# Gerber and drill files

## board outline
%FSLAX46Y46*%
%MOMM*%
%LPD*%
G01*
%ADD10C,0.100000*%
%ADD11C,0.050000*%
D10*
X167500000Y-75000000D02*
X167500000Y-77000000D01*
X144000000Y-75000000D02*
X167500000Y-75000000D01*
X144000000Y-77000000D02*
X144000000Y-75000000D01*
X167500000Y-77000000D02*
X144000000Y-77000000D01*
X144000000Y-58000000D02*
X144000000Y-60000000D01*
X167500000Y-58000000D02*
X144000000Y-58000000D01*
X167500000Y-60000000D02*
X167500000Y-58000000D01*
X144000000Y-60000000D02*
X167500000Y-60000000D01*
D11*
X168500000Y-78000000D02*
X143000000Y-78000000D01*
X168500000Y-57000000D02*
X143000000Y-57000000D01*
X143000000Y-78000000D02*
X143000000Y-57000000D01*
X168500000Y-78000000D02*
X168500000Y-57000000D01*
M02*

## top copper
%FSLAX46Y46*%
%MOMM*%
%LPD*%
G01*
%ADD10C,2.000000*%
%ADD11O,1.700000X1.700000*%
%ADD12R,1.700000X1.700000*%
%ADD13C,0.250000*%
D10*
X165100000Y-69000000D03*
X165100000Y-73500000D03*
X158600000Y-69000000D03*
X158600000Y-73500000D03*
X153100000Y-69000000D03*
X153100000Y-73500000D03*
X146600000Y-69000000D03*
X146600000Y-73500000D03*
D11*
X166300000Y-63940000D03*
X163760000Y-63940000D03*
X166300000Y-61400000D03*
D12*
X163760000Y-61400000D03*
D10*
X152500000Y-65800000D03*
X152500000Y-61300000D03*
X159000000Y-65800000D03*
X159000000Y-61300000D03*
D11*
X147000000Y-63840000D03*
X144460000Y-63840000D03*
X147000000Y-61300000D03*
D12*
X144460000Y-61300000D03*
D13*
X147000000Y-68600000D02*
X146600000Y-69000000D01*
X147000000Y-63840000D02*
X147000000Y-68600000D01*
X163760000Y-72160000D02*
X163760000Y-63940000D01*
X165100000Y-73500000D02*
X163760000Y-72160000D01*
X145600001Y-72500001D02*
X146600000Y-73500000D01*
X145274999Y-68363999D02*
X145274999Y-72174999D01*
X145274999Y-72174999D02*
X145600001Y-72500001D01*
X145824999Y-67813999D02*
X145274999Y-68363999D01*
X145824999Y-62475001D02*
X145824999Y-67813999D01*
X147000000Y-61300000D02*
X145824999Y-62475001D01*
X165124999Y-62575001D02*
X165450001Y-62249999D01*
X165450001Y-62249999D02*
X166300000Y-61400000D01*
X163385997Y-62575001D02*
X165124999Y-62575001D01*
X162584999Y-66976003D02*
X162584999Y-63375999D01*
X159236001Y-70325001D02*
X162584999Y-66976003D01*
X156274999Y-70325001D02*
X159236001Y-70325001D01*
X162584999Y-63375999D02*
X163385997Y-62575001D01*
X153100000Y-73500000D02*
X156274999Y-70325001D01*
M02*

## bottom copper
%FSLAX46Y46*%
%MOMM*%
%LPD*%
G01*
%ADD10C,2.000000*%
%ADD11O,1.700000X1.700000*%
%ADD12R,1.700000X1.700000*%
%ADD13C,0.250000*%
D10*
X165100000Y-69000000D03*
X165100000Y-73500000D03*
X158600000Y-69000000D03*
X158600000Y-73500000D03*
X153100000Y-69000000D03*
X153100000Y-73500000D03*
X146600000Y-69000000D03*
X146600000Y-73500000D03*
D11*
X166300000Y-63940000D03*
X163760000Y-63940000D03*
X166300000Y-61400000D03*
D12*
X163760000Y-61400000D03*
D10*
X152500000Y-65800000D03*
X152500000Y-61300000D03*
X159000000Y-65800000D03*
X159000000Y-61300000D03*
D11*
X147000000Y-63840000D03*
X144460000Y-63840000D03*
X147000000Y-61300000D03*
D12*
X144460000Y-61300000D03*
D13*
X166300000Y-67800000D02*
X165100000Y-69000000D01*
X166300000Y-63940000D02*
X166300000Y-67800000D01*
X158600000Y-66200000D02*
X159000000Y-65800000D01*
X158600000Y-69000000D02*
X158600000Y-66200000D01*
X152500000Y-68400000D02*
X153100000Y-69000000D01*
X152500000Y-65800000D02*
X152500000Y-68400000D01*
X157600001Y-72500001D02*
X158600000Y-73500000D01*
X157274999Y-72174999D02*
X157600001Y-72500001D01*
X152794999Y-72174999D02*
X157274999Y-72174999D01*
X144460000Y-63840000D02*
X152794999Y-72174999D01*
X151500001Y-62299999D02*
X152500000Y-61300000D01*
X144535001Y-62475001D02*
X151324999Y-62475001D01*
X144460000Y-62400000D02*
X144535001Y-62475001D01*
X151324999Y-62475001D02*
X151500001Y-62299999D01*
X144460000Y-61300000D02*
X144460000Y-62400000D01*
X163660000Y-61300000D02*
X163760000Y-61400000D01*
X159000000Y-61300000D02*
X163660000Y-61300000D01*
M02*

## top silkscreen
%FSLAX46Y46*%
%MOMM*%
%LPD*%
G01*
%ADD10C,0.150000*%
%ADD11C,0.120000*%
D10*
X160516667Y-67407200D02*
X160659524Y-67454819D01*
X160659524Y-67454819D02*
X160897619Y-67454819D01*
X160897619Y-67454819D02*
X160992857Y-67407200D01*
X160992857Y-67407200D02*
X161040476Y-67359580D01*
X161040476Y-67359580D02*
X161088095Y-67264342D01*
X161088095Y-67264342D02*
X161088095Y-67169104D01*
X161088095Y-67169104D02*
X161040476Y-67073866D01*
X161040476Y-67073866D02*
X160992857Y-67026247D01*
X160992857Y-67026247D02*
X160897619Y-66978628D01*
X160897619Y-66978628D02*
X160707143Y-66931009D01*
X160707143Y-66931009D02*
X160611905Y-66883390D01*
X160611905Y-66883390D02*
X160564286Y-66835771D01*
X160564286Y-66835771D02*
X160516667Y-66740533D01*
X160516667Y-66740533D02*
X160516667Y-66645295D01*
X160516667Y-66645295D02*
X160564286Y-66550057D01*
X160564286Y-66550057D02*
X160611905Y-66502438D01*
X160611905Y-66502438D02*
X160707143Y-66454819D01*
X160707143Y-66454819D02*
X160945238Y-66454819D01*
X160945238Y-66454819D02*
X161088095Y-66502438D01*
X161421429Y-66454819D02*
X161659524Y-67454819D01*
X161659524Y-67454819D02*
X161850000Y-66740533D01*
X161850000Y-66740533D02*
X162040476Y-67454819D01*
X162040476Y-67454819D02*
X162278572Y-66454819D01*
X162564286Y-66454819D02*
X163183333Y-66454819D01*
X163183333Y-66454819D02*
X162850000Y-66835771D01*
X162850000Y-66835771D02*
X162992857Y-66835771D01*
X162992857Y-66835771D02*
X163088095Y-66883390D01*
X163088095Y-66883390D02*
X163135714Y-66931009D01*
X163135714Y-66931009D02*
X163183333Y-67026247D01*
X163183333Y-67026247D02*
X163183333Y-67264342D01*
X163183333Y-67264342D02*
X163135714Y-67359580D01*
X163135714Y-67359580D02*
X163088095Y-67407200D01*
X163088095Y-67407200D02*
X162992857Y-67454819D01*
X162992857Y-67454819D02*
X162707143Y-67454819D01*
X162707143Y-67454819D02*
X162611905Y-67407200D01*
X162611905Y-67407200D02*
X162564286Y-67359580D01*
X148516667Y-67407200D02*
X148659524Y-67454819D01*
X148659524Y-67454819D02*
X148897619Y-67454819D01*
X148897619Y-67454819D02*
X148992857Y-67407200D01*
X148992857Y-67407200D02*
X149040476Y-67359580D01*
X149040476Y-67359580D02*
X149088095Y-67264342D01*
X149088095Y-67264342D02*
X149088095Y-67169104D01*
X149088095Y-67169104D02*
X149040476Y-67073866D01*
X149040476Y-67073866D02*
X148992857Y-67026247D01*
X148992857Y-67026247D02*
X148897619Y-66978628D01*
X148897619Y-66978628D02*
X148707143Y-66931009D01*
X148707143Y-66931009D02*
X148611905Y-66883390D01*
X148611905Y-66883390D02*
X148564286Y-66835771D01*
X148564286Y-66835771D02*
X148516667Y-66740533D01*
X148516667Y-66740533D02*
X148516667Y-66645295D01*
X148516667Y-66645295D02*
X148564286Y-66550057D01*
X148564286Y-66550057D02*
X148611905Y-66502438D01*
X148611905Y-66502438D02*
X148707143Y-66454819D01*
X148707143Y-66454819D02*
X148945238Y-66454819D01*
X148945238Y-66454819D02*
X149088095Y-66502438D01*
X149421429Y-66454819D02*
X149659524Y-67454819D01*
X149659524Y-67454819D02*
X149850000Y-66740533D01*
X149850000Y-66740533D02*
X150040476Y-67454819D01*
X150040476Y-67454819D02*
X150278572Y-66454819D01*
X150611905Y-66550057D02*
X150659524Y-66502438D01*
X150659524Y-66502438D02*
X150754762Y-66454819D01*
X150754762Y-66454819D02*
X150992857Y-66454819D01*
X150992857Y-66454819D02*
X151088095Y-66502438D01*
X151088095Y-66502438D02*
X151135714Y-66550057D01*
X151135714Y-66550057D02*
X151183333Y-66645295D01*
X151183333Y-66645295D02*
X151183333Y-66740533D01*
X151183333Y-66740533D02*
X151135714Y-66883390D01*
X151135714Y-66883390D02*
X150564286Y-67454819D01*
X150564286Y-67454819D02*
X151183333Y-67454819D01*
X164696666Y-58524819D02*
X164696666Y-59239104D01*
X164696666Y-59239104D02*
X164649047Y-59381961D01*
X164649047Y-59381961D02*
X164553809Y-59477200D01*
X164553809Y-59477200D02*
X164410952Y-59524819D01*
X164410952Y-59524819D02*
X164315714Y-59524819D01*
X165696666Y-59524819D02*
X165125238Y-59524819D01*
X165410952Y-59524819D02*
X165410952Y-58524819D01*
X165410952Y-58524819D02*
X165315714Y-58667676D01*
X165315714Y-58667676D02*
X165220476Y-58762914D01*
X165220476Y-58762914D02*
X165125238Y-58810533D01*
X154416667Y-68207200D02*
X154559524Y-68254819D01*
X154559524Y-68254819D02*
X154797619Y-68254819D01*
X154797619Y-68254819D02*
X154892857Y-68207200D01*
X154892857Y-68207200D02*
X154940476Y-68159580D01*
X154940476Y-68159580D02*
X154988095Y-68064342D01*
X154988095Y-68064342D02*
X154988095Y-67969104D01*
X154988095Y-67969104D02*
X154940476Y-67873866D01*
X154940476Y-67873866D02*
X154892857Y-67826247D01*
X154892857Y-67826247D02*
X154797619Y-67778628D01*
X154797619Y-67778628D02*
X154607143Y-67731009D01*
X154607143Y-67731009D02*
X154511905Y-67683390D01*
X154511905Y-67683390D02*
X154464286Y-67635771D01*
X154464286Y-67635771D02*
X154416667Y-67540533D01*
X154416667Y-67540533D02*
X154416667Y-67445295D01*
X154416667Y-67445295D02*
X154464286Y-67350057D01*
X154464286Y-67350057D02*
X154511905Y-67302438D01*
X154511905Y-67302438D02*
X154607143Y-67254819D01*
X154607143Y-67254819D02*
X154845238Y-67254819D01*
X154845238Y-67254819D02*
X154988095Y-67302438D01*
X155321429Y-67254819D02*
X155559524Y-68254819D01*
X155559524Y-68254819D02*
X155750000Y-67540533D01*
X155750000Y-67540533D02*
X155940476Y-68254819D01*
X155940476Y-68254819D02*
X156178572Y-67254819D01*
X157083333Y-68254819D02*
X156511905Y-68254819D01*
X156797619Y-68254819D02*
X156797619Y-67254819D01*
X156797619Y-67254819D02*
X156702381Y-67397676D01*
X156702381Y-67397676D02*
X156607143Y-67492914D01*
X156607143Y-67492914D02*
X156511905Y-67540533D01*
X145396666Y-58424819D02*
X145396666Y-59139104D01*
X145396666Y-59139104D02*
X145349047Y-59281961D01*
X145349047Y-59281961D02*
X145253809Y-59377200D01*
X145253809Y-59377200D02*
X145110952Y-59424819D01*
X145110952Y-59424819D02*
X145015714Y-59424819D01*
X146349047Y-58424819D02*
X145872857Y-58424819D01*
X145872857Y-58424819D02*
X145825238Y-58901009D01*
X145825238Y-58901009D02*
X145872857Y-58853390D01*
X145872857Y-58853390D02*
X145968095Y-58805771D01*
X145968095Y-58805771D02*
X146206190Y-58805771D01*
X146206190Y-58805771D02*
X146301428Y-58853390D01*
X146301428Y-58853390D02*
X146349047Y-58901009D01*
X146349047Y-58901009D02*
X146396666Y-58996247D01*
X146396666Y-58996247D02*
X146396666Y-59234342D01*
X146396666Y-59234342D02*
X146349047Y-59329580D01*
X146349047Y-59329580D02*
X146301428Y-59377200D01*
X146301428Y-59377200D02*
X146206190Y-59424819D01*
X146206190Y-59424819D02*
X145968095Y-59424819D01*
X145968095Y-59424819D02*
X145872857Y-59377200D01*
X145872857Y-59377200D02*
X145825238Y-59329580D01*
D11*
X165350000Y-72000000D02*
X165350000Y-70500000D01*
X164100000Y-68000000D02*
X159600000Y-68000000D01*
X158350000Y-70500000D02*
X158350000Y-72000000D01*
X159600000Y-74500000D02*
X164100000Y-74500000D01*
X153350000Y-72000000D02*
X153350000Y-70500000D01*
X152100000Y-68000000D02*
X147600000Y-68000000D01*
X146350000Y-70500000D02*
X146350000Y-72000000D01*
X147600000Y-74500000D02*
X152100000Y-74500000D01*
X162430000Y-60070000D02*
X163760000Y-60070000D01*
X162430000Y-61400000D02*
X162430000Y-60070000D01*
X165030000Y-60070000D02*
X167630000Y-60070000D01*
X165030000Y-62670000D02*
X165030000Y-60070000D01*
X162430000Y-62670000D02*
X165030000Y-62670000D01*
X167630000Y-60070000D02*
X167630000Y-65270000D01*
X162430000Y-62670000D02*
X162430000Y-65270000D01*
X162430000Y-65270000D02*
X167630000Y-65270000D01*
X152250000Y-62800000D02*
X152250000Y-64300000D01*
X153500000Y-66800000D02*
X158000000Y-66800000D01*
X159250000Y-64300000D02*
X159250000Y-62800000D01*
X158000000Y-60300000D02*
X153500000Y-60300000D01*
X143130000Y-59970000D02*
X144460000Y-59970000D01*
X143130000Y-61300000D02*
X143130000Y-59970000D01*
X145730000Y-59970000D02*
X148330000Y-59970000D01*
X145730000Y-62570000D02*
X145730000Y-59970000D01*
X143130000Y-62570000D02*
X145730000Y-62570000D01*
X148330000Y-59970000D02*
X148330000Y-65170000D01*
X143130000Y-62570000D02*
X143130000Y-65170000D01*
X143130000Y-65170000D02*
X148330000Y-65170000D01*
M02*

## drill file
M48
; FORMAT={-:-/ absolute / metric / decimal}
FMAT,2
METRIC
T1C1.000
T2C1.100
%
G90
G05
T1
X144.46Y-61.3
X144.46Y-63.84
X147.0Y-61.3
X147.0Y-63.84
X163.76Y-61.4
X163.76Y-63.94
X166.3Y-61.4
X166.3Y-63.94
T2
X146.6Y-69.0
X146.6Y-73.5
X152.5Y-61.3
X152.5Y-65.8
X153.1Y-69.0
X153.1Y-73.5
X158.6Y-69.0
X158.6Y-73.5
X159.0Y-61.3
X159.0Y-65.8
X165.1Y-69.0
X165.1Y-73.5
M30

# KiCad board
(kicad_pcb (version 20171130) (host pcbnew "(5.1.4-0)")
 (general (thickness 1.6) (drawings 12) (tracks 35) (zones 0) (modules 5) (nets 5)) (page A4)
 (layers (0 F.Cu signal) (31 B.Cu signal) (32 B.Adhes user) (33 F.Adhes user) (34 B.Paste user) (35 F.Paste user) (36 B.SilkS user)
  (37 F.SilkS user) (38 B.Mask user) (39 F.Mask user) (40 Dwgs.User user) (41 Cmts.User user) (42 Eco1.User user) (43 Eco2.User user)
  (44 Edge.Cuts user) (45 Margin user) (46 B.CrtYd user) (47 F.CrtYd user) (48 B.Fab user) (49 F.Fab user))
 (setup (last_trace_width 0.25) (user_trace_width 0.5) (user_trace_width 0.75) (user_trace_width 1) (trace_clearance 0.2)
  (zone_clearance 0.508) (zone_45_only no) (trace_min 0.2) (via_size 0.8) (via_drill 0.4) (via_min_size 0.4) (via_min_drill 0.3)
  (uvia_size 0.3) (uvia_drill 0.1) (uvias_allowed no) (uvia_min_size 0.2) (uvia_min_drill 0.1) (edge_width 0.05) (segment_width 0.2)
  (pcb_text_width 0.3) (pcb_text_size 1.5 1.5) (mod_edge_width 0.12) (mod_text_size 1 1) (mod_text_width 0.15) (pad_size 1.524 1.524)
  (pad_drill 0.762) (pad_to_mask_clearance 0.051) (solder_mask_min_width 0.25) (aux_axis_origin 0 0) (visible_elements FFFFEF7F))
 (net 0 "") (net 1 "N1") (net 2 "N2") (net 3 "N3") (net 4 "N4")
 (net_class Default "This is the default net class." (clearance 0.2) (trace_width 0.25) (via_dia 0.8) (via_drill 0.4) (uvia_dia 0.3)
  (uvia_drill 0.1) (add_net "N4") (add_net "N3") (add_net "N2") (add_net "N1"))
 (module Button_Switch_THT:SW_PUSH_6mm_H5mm (layer F.Cu) (at 158.6 69)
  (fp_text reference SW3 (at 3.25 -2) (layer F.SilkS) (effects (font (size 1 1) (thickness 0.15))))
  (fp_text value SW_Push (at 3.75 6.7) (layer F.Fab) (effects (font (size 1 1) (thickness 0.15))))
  (fp_line (start 6.75 3) (end 6.75 1.5) (layer F.SilkS) (width 0.12))
  (fp_line (start 5.5 -1) (end 1 -1) (layer F.SilkS) (width 0.12))
  (fp_line (start -0.25 1.5) (end -0.25 3) (layer F.SilkS) (width 0.12))
  (fp_line (start 1 5.5) (end 5.5 5.5) (layer F.SilkS) (width 0.12))
  (pad 1 thru_hole circle (at 6.5 0 90) (size 2 2) (drill 1.1) (layers *.Cu *.Mask) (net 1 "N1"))
  (pad 2 thru_hole circle (at 6.5 4.5 90) (size 2 2) (drill 1.1) (layers *.Cu *.Mask) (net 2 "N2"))
  (pad 1 thru_hole circle (at 0 0 90) (size 2 2) (drill 1.1) (layers *.Cu *.Mask) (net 1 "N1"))
  (pad 2 thru_hole circle (at 0 4.5 90) (size 2 2) (drill 1.1) (layers *.Cu *.Mask) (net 2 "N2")))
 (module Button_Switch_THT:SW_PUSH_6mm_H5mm (layer F.Cu) (at 146.6 69)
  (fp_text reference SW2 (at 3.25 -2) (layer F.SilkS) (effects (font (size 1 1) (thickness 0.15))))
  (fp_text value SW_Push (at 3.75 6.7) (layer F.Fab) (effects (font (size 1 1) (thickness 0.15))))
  (fp_line (start 6.75 3) (end 6.75 1.5) (layer F.SilkS) (width 0.12))
  (fp_line (start 5.5 -1) (end 1 -1) (layer F.SilkS) (width 0.12))
  (fp_line (start -0.25 1.5) (end -0.25 3) (layer F.SilkS) (width 0.12))
  (fp_line (start 1 5.5) (end 5.5 5.5) (layer F.SilkS) (width 0.12))
  (pad 1 thru_hole circle (at 6.5 0 90) (size 2 2) (drill 1.1) (layers *.Cu *.Mask) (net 1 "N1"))
  (pad 2 thru_hole circle (at 6.5 4.5 90) (size 2 2) (drill 1.1) (layers *.Cu *.Mask) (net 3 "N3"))
  (pad 1 thru_hole circle (at 0 0 90) (size 2 2) (drill 1.1) (layers *.Cu *.Mask) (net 1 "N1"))
  (pad 2 thru_hole circle (at 0 4.5 90) (size 2 2) (drill 1.1) (layers *.Cu *.Mask) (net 3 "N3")))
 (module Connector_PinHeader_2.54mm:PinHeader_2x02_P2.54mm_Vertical (layer F.Cu) (at 163.76 61.4)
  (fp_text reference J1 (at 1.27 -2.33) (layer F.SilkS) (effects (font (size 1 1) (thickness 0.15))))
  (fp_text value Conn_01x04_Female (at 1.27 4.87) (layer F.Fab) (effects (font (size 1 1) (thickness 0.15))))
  (fp_line (start -1.33 -1.33) (end 0 -1.33) (layer F.SilkS) (width 0.12))
  (fp_line (start -1.33 0) (end -1.33 -1.33) (layer F.SilkS) (width 0.12))
  (fp_line (start 1.27 -1.33) (end 3.87 -1.33) (layer F.SilkS) (width 0.12))
  (fp_line (start 1.27 1.27) (end 1.27 -1.33) (layer F.SilkS) (width 0.12))
  (fp_line (start -1.33 1.27) (end 1.27 1.27) (layer F.SilkS) (width 0.12))
  (fp_line (start 3.87 -1.33) (end 3.87 3.87) (layer F.SilkS) (width 0.12))
  (fp_line (start -1.33 1.27) (end -1.33 3.87) (layer F.SilkS) (width 0.12))
  (fp_line (start -1.33 3.87) (end 3.87 3.87) (layer F.SilkS) (width 0.12))
  (pad 4 thru_hole oval (at 2.54 2.54) (size 1.7 1.7) (drill 1) (layers *.Cu *.Mask) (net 1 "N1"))
  (pad 3 thru_hole oval (at 0 2.54) (size 1.7 1.7) (drill 1) (layers *.Cu *.Mask) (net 2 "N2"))
  (pad 2 thru_hole oval (at 2.54 0) (size 1.7 1.7) (drill 1) (layers *.Cu *.Mask) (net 3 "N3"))
  (pad 1 thru_hole rect (at 0 0) (size 1.7 1.7) (drill 1) (layers *.Cu *.Mask) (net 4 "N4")))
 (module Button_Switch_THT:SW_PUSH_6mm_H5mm (layer F.Cu) (at 159 65.8 180)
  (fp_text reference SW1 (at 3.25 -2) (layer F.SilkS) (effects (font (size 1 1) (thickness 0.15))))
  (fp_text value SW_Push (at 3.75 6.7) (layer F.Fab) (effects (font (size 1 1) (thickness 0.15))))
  (fp_line (start 6.75 3) (end 6.75 1.5) (layer F.SilkS) (width 0.12))
  (fp_line (start 5.5 -1) (end 1 -1) (layer F.SilkS) (width 0.12))
  (fp_line (start -0.25 1.5) (end -0.25 3) (layer F.SilkS) (width 0.12))
  (fp_line (start 1 5.5) (end 5.5 5.5) (layer F.SilkS) (width 0.12))
  (pad 1 thru_hole circle (at 6.5 0 270) (size 2 2) (drill 1.1) (layers *.Cu *.Mask) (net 1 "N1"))
  (pad 2 thru_hole circle (at 6.5 4.5 270) (size 2 2) (drill 1.1) (layers *.Cu *.Mask) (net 4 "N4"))
  (pad 1 thru_hole circle (at 0 0 270) (size 2 2) (drill 1.1) (layers *.Cu *.Mask) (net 1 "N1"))
  (pad 2 thru_hole circle (at 0 4.5 270) (size 2 2) (drill 1.1) (layers *.Cu *.Mask) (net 4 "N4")))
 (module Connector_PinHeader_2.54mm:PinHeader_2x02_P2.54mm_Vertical (layer F.Cu) (at 144.46 61.3)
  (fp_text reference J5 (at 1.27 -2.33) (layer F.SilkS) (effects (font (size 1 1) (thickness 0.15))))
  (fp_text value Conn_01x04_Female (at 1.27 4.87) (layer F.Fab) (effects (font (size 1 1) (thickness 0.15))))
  (fp_line (start -1.33 -1.33) (end 0 -1.33) (layer F.SilkS) (width 0.12))
  (fp_line (start -1.33 0) (end -1.33 -1.33) (layer F.SilkS) (width 0.12))
  (fp_line (start 1.27 -1.33) (end 3.87 -1.33) (layer F.SilkS) (width 0.12))
  (fp_line (start 1.27 1.27) (end 1.27 -1.33) (layer F.SilkS) (width 0.12))
  (fp_line (start -1.33 1.27) (end 1.27 1.27) (layer F.SilkS) (width 0.12))
  (fp_line (start 3.87 -1.33) (end 3.87 3.87) (layer F.SilkS) (width 0.12))
  (fp_line (start -1.33 1.27) (end -1.33 3.87) (layer F.SilkS) (width 0.12))
  (fp_line (start -1.33 3.87) (end 3.87 3.87) (layer F.SilkS) (width 0.12))
  (pad 4 thru_hole oval (at 2.54 2.54) (size 1.7 1.7) (drill 1) (layers *.Cu *.Mask) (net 1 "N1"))
  (pad 3 thru_hole oval (at 0 2.54) (size 1.7 1.7) (drill 1) (layers *.Cu *.Mask) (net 2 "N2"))
  (pad 2 thru_hole oval (at 2.54 0) (size 1.7 1.7) (drill 1) (layers *.Cu *.Mask) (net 3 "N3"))
  (pad 1 thru_hole rect (at 0 0) (size 1.7 1.7) (drill 1) (layers *.Cu *.Mask) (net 4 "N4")))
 (gr_line (start 167.5 75) (end 167.5 77) (layer Edge.Cuts) (width 0.1))
 (gr_line (start 144 75) (end 167.5 75) (layer Edge.Cuts) (width 0.1))
 (gr_line (start 144 77) (end 144 75) (layer Edge.Cuts) (width 0.1))
 (gr_line (start 167.5 77) (end 144 77) (layer Edge.Cuts) (width 0.1))
 (gr_line (start 144 58) (end 144 60) (layer Edge.Cuts) (width 0.1))
 (gr_line (start 167.5 58) (end 144 58) (layer Edge.Cuts) (width 0.1))
 (gr_line (start 167.5 60) (end 167.5 58) (layer Edge.Cuts) (width 0.1))
 (gr_line (start 144 60) (end 167.5 60) (layer Edge.Cuts) (width 0.1))
 (gr_line (start 168.5 78) (end 143 78) (layer Edge.Cuts) (width 0.05))
 (gr_line (start 168.5 57) (end 143 57) (layer Edge.Cuts) (width 0.05))
 (gr_line (start 143 78) (end 143 57) (layer Edge.Cuts) (width 0.05))
 (gr_line (start 168.5 78) (end 168.5 57) (layer Edge.Cuts) (width 0.05))
 (segment (start 166.3 67.8) (end 165.1 69) (width 0.25) (layer B.Cu) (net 1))
 (segment (start 166.3 63.94) (end 166.3 67.8) (width 0.25) (layer B.Cu) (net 1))
 (segment (start 158.6 66.2) (end 159 65.8) (width 0.25) (layer B.Cu) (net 1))
 (segment (start 158.6 69) (end 158.6 66.2) (width 0.25) (layer B.Cu) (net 1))
 (segment (start 152.5 68.4) (end 153.1 69) (width 0.25) (layer B.Cu) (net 1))
 (segment (start 152.5 65.8) (end 152.5 68.4) (width 0.25) (layer B.Cu) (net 1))
 (segment (start 147 68.6) (end 146.6 69) (width 0.25) (layer F.Cu) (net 1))
 (segment (start 147 63.84) (end 147 68.6) (width 0.25) (layer F.Cu) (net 1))
 (segment (start 163.76 72.16) (end 163.76 63.94) (width 0.25) (layer F.Cu) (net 2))
 (segment (start 165.1 73.5) (end 163.76 72.16) (width 0.25) (layer F.Cu) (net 2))
 (segment (start 157.600001 72.500001) (end 158.6 73.5) (width 0.25) (layer B.Cu) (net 2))
 (segment (start 157.274999 72.174999) (end 157.600001 72.500001) (width 0.25) (layer B.Cu) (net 2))
 (segment (start 152.794999 72.174999) (end 157.274999 72.174999) (width 0.25) (layer B.Cu) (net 2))
 (segment (start 144.46 63.84) (end 152.794999 72.174999) (width 0.25) (layer B.Cu) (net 2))
 (segment (start 145.600001 72.500001) (end 146.6 73.5) (width 0.25) (layer F.Cu) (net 3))
 (segment (start 145.274999 68.363999) (end 145.274999 72.174999) (width 0.25) (layer F.Cu) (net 3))
 (segment (start 145.274999 72.174999) (end 145.600001 72.500001) (width 0.25) (layer F.Cu) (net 3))
 (segment (start 145.824999 67.813999) (end 145.274999 68.363999) (width 0.25) (layer F.Cu) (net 3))
 (segment (start 145.824999 62.475001) (end 145.824999 67.813999) (width 0.25) (layer F.Cu) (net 3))
 (segment (start 147 61.3) (end 145.824999 62.475001) (width 0.25) (layer F.Cu) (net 3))
 (segment (start 165.124999 62.575001) (end 165.450001 62.249999) (width 0.25) (layer F.Cu) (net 3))
 (segment (start 165.450001 62.249999) (end 166.3 61.4) (width 0.25) (layer F.Cu) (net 3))
 (segment (start 163.385997 62.575001) (end 165.124999 62.575001) (width 0.25) (layer F.Cu) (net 3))
 (segment (start 162.584999 66.976003) (end 162.584999 63.375999) (width 0.25) (layer F.Cu) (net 3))
 (segment (start 159.236001 70.325001) (end 162.584999 66.976003) (width 0.25) (layer F.Cu) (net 3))
 (segment (start 156.274999 70.325001) (end 159.236001 70.325001) (width 0.25) (layer F.Cu) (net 3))
 (segment (start 162.584999 63.375999) (end 163.385997 62.575001) (width 0.25) (layer F.Cu) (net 3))
 (segment (start 153.1 73.5) (end 156.274999 70.325001) (width 0.25) (layer F.Cu) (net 3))
 (segment (start 151.500001 62.299999) (end 152.5 61.3) (width 0.25) (layer B.Cu) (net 4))
 (segment (start 144.535001 62.475001) (end 151.324999 62.475001) (width 0.25) (layer B.Cu) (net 4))
 (segment (start 144.46 62.4) (end 144.535001 62.475001) (width 0.25) (layer B.Cu) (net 4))
 (segment (start 151.324999 62.475001) (end 151.500001 62.299999) (width 0.25) (layer B.Cu) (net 4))
 (segment (start 144.46 61.3) (end 144.46 62.4) (width 0.25) (layer B.Cu) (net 4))
 (segment (start 163.66 61.3) (end 163.76 61.4) (width 0.25) (layer B.Cu) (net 4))
 (segment (start 159 61.3) (end 163.66 61.3) (width 0.25) (layer B.Cu) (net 4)))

